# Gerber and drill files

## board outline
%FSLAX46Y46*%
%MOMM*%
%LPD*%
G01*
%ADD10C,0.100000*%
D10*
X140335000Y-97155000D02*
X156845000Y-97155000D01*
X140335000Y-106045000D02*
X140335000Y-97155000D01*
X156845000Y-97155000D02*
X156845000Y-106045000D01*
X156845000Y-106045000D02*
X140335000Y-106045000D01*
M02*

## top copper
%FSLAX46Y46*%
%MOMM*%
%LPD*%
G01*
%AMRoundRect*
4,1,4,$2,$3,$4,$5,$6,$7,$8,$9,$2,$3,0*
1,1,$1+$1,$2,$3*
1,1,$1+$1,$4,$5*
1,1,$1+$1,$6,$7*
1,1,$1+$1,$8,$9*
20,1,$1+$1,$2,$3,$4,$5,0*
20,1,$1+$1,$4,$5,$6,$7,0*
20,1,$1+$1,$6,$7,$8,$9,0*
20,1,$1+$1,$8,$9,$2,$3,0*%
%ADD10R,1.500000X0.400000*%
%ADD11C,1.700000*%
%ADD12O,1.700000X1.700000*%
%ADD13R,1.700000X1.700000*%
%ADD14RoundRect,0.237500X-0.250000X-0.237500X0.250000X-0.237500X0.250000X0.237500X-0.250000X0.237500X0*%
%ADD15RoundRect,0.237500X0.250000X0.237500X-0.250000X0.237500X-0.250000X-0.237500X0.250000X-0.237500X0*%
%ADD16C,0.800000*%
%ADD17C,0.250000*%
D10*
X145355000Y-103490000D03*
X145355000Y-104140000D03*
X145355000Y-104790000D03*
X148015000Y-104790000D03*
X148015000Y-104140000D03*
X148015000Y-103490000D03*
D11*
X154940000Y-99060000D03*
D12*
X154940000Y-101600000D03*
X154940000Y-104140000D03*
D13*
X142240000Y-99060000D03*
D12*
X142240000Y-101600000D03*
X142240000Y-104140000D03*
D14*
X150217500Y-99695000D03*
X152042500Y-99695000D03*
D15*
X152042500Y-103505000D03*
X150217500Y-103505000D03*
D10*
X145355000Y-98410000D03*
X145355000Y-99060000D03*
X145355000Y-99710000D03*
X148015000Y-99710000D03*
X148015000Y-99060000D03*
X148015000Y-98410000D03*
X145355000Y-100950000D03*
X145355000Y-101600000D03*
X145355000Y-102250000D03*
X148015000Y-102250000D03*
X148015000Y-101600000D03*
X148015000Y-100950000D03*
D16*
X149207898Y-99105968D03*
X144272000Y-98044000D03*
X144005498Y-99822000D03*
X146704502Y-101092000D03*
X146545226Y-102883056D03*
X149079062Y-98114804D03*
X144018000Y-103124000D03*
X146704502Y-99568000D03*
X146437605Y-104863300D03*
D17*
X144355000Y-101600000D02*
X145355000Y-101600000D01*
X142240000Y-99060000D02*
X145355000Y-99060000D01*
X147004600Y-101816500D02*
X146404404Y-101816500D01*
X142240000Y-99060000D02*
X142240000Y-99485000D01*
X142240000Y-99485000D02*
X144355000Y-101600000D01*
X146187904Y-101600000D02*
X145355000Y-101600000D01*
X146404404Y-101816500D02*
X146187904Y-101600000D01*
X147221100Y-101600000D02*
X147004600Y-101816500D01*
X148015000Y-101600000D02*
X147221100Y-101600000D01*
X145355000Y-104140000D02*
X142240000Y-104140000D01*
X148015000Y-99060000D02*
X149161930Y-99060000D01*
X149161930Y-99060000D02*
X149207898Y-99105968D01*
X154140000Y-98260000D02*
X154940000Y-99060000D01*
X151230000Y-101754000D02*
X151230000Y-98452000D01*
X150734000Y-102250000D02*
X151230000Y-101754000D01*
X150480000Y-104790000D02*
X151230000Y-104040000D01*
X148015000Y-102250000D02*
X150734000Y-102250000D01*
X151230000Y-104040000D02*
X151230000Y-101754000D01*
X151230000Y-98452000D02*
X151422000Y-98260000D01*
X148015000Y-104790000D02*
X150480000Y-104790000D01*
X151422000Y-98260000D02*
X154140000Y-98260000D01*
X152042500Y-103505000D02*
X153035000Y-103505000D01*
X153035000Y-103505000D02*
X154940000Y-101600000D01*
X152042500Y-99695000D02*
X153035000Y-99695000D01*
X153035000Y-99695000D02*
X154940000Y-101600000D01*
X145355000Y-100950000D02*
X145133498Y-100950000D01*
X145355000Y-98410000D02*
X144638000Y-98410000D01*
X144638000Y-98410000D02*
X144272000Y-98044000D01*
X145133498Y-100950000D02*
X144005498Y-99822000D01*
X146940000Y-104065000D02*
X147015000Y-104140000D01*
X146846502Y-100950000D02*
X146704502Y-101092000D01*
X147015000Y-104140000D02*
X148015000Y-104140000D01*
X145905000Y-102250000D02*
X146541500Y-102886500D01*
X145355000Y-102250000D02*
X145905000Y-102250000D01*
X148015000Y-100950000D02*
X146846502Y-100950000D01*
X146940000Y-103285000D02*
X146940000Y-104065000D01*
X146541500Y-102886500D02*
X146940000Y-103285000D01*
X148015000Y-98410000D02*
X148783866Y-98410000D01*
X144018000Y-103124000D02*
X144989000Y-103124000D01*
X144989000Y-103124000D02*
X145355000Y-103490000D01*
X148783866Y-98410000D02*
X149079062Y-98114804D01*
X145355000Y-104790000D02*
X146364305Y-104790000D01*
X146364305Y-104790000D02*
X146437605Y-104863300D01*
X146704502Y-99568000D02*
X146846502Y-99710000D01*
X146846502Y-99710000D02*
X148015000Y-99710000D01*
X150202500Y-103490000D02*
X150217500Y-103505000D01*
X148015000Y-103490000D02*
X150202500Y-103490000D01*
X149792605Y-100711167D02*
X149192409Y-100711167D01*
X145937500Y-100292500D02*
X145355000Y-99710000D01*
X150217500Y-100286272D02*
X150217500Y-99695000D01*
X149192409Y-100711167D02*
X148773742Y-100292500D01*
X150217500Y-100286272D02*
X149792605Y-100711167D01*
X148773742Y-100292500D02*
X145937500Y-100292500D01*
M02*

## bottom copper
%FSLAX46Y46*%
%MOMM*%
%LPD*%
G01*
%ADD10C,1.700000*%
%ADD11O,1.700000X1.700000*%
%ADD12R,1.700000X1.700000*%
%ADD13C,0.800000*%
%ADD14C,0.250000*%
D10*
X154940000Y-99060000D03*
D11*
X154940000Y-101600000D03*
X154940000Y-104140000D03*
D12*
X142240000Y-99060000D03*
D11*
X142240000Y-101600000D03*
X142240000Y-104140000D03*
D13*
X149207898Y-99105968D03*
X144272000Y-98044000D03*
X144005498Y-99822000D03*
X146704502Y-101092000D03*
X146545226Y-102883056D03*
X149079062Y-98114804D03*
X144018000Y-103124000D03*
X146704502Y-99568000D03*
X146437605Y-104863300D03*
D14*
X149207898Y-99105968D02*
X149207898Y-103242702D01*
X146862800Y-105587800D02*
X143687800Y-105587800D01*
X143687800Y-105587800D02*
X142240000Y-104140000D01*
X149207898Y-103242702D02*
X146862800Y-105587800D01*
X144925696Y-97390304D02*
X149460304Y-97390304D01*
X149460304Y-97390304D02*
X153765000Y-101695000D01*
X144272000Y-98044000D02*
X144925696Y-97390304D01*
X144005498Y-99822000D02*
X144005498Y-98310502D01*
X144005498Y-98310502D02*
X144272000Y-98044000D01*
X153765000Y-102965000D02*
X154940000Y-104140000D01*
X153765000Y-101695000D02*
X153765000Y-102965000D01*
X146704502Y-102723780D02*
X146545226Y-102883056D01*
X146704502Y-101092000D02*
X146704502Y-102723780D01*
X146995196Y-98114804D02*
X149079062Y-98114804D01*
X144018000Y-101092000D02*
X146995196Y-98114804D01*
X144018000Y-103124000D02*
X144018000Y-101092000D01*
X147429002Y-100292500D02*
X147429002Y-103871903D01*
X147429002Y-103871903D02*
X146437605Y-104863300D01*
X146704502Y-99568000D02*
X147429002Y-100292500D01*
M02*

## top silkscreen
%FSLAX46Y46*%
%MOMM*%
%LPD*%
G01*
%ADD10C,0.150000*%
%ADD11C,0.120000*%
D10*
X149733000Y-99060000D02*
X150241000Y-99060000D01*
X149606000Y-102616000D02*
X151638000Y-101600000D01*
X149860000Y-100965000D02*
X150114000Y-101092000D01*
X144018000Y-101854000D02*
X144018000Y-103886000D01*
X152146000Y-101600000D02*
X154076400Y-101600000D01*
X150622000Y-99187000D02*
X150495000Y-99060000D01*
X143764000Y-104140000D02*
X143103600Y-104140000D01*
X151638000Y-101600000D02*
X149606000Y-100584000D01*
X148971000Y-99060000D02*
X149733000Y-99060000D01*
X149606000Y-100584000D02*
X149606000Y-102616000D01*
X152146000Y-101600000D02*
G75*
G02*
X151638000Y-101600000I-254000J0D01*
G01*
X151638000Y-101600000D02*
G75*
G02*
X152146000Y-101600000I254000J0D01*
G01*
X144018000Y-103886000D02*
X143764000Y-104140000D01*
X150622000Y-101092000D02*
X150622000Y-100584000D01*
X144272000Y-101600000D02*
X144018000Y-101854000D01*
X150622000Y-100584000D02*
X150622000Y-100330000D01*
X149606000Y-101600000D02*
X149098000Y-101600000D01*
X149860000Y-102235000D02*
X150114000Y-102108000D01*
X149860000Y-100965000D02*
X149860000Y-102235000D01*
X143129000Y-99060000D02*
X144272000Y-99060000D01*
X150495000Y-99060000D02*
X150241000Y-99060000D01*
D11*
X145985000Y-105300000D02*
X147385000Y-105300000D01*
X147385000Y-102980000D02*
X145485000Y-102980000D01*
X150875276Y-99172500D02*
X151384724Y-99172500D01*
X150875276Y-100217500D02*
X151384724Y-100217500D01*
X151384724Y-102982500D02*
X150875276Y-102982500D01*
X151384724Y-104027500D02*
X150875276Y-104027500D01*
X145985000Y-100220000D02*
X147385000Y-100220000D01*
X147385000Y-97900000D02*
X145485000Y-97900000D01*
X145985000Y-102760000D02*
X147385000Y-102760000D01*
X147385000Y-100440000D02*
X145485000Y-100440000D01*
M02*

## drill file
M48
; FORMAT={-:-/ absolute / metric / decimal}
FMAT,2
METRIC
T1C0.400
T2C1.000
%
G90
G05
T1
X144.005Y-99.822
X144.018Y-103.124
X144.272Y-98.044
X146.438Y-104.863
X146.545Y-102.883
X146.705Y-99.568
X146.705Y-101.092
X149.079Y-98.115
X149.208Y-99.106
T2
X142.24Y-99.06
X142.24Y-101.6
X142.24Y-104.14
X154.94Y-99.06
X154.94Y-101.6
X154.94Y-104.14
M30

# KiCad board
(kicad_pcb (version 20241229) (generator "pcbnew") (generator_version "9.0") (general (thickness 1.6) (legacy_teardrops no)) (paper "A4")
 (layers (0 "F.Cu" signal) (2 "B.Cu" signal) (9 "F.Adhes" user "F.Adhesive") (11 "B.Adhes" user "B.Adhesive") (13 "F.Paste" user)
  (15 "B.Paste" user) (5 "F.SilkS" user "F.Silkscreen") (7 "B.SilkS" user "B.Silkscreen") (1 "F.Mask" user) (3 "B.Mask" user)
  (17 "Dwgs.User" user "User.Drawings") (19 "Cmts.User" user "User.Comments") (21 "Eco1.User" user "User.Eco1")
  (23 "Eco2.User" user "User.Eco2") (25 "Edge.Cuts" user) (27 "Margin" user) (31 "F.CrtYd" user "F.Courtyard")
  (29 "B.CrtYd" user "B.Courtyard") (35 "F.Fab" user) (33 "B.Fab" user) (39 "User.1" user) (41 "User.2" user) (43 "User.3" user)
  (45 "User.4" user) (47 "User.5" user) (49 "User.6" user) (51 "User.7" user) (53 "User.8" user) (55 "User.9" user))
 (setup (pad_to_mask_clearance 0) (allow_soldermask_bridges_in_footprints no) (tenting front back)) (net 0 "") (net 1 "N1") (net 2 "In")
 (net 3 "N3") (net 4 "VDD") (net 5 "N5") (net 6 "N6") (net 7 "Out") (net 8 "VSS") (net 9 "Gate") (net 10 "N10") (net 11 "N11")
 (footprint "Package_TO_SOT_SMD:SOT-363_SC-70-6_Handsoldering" (layer "F.Cu") (at 146.685 104.14)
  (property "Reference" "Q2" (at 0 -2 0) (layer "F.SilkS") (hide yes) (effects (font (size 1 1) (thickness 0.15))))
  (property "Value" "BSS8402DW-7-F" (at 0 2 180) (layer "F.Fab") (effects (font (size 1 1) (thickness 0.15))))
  (fp_line (start -0.7 1.16) (end 0.7 1.16) (stroke (width 0.12) (type solid)) (layer "F.SilkS"))
  (fp_line (start 0.7 -1.16) (end -1.2 -1.16) (stroke (width 0.12) (type solid)) (layer "F.SilkS"))
  (pad "1" smd rect (at -1.33 -0.65) (size 1.5 0.4) (layers "F.Cu" "F.Mask" "F.Paste") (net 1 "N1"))
  (pad "2" smd rect (at -1.33 0) (size 1.5 0.4) (layers "F.Cu" "F.Mask" "F.Paste") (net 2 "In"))
  (pad "3" smd rect (at -1.33 0.65) (size 1.5 0.4) (layers "F.Cu" "F.Mask" "F.Paste") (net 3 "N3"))
  (pad "4" smd rect (at 1.33 0.65) (size 1.5 0.4) (layers "F.Cu" "F.Mask" "F.Paste") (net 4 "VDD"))
  (pad "5" smd rect (at 1.33 0) (size 1.5 0.4) (layers "F.Cu" "F.Mask" "F.Paste") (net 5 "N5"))
  (pad "6" smd rect (at 1.33 -0.65) (size 1.5 0.4) (layers "F.Cu" "F.Mask" "F.Paste") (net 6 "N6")))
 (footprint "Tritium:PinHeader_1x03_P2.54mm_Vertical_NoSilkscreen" (layer "F.Cu") (at 154.94 99.06)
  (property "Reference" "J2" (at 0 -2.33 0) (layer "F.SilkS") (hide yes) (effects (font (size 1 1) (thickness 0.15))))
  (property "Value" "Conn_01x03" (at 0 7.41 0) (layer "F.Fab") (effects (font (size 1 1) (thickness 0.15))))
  (pad "1" thru_hole circle (at 0 0) (size 1.7 1.7) (drill 1) (layers "*.Cu" "*.Mask") (remove_unused_layers no) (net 4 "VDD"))
  (pad "2" thru_hole oval (at 0 2.54) (size 1.7 1.7) (drill 1) (layers "*.Cu" "*.Mask") (remove_unused_layers no) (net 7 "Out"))
  (pad "3" thru_hole oval (at 0 5.08) (size 1.7 1.7) (drill 1) (layers "*.Cu" "*.Mask") (remove_unused_layers no) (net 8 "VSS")))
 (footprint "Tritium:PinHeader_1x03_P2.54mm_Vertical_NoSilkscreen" (layer "F.Cu") (at 142.24 99.06)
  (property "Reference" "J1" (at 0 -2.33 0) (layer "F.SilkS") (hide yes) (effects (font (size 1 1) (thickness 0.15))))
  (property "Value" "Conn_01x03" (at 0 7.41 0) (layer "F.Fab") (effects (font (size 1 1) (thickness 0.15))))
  (pad "1" thru_hole rect (at 0 0) (size 1.7 1.7) (drill 1) (layers "*.Cu" "*.Mask") (remove_unused_layers no) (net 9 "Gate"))
  (pad "2" thru_hole oval (at 0 2.54) (size 1.7 1.7) (drill 1) (layers "*.Cu" "*.Mask") (remove_unused_layers no) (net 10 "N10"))
  (pad "3" thru_hole oval (at 0 5.08) (size 1.7 1.7) (drill 1) (layers "*.Cu" "*.Mask") (remove_unused_layers no) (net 2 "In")))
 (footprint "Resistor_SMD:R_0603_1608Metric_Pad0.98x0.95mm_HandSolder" (layer "F.Cu") (at 151.13 99.695)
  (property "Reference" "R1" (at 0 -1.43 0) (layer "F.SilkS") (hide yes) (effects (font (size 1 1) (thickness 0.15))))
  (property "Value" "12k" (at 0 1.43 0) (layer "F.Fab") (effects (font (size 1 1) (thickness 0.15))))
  (fp_line (start -0.254724 -0.5225) (end 0.254724 -0.5225) (stroke (width 0.12) (type solid)) (layer "F.SilkS"))
  (fp_line (start -0.254724 0.5225) (end 0.254724 0.5225) (stroke (width 0.12) (type solid)) (layer "F.SilkS"))
  (pad "1" smd roundrect (at -0.9125 0) (size 0.975 0.95) (layers "F.Cu" "F.Mask" "F.Paste") (roundrect_rratio 0.25) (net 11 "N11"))
  (pad "2" smd roundrect (at 0.9125 0) (size 0.975 0.95) (layers "F.Cu" "F.Mask" "F.Paste") (roundrect_rratio 0.25) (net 7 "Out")))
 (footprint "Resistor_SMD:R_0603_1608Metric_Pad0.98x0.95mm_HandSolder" (layer "F.Cu") (at 151.13 103.505 180)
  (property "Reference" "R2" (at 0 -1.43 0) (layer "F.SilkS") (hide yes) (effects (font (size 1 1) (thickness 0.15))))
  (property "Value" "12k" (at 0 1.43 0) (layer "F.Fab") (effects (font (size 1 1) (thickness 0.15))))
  (fp_line (start -0.254724 0.5225) (end 0.254724 0.5225) (stroke (width 0.12) (type solid)) (layer "F.SilkS"))
  (fp_line (start -0.254724 -0.5225) (end 0.254724 -0.5225) (stroke (width 0.12) (type solid)) (layer "F.SilkS"))
  (pad "1" smd roundrect (at -0.9125 0 180) (size 0.975 0.95) (layers "F.Cu" "F.Mask" "F.Paste") (roundrect_rratio 0.25) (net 7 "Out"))
  (pad "2" smd roundrect (at 0.9125 0 180) (size 0.975 0.95) (layers "F.Cu" "F.Mask" "F.Paste") (roundrect_rratio 0.25) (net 6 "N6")))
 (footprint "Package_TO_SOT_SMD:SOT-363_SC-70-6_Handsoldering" (layer "F.Cu") (at 146.685 99.06)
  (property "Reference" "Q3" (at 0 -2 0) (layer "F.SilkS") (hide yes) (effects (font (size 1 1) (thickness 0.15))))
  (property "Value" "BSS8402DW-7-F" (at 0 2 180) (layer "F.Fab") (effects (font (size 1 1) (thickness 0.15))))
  (fp_line (start -0.7 1.16) (end 0.7 1.16) (stroke (width 0.12) (type solid)) (layer "F.SilkS"))
  (fp_line (start 0.7 -1.16) (end -1.2 -1.16) (stroke (width 0.12) (type solid)) (layer "F.SilkS"))
  (pad "1" smd rect (at -1.33 -0.65) (size 1.5 0.4) (layers "F.Cu" "F.Mask" "F.Paste") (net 8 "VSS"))
  (pad "2" smd rect (at -1.33 0) (size 1.5 0.4) (layers "F.Cu" "F.Mask" "F.Paste") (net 9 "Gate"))
  (pad "3" smd rect (at -1.33 0.65) (size 1.5 0.4) (layers "F.Cu" "F.Mask" "F.Paste") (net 11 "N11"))
  (pad "4" smd rect (at 1.33 0.65) (size 1.5 0.4) (layers "F.Cu" "F.Mask" "F.Paste") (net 3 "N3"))
  (pad "5" smd rect (at 1.33 0) (size 1.5 0.4) (layers "F.Cu" "F.Mask" "F.Paste") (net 2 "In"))
  (pad "6" smd rect (at 1.33 -0.65) (size 1.5 0.4) (layers "F.Cu" "F.Mask" "F.Paste") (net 1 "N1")))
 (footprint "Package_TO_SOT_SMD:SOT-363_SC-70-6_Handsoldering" (layer "F.Cu") (at 146.685 101.6)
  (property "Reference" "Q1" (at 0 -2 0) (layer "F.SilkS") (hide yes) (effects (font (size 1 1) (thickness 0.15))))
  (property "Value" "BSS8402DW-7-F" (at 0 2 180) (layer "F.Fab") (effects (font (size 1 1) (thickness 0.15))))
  (fp_line (start -0.7 1.16) (end 0.7 1.16) (stroke (width 0.12) (type solid)) (layer "F.SilkS"))
  (fp_line (start 0.7 -1.16) (end -1.2 -1.16) (stroke (width 0.12) (type solid)) (layer "F.SilkS"))
  (pad "1" smd rect (at -1.33 -0.65) (size 1.5 0.4) (layers "F.Cu" "F.Mask" "F.Paste") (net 8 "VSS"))
  (pad "2" smd rect (at -1.33 0) (size 1.5 0.4) (layers "F.Cu" "F.Mask" "F.Paste") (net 9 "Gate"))
  (pad "3" smd rect (at -1.33 0.65) (size 1.5 0.4) (layers "F.Cu" "F.Mask" "F.Paste") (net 5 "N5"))
  (pad "4" smd rect (at 1.33 0.65) (size 1.5 0.4) (layers "F.Cu" "F.Mask" "F.Paste") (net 4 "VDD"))
  (pad "5" smd rect (at 1.33 0) (size 1.5 0.4) (layers "F.Cu" "F.Mask" "F.Paste") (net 9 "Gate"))
  (pad "6" smd rect (at 1.33 -0.65) (size 1.5 0.4) (layers "F.Cu" "F.Mask" "F.Paste") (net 5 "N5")))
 (gr_line (start 149.733 99.06) (end 150.241 99.06) (stroke (width 0.15) (type solid)) (layer "F.SilkS"))
 (gr_line (start 149.606 102.616) (end 151.638 101.6) (stroke (width 0.15) (type solid)) (layer "F.SilkS"))
 (gr_line (start 149.86 100.965) (end 150.114 101.092) (stroke (width 0.15) (type solid)) (layer "F.SilkS"))
 (gr_line (start 144.018 101.854) (end 144.018 103.886) (stroke (width 0.15) (type solid)) (layer "F.SilkS"))
 (gr_line (start 152.146 101.6) (end 154.0764 101.6) (stroke (width 0.15) (type solid)) (layer "F.SilkS"))
 (gr_line (start 150.622 99.187) (end 150.495 99.06) (stroke (width 0.15) (type solid)) (layer "F.SilkS"))
 (gr_line (start 143.764 104.14) (end 143.1036 104.14) (stroke (width 0.15) (type solid)) (layer "F.SilkS"))
 (gr_line (start 151.638 101.6) (end 149.606 100.584) (stroke (width 0.15) (type solid)) (layer "F.SilkS"))
 (gr_line (start 148.971 99.06) (end 149.733 99.06) (stroke (width 0.15) (type solid)) (layer "F.SilkS"))
 (gr_line (start 149.606 100.584) (end 149.606 102.616) (stroke (width 0.15) (type solid)) (layer "F.SilkS"))
 (gr_circle (center 151.892 101.6) (end 152.146 101.6) (stroke (width 0.15) (type solid)) (fill no) (layer "F.SilkS"))
 (gr_line (start 144.018 103.886) (end 143.764 104.14) (stroke (width 0.15) (type solid)) (layer "F.SilkS"))
 (gr_line (start 150.622 101.092) (end 150.622 100.584) (stroke (width 0.15) (type solid)) (layer "F.SilkS"))
 (gr_line (start 144.272 101.6) (end 144.018 101.854) (stroke (width 0.15) (type solid)) (layer "F.SilkS"))
 (gr_line (start 150.622 100.584) (end 150.622 100.33) (stroke (width 0.15) (type solid)) (layer "F.SilkS"))
 (gr_line (start 149.606 101.6) (end 149.098 101.6) (stroke (width 0.15) (type solid)) (layer "F.SilkS"))
 (gr_line (start 149.86 102.235) (end 150.114 102.108) (stroke (width 0.15) (type solid)) (layer "F.SilkS"))
 (gr_line (start 149.86 100.965) (end 149.86 102.235) (stroke (width 0.15) (type solid)) (layer "F.SilkS"))
 (gr_line (start 143.129 99.06) (end 144.272 99.06) (stroke (width 0.15) (type solid)) (layer "F.SilkS"))
 (gr_line (start 150.495 99.06) (end 150.241 99.06) (stroke (width 0.15) (type solid)) (layer "F.SilkS"))
 (gr_line (start 140.335 97.155) (end 156.845 97.155) (stroke (width 0.1) (type solid)) (layer "Edge.Cuts"))
 (gr_line (start 140.335 106.045) (end 140.335 97.155) (stroke (width 0.1) (type solid)) (layer "Edge.Cuts"))
 (gr_line (start 156.845 97.155) (end 156.845 106.045) (stroke (width 0.1) (type solid)) (layer "Edge.Cuts"))
 (gr_line (start 156.845 106.045) (end 140.335 106.045) (stroke (width 0.1) (type solid)) (layer "Edge.Cuts"))
 (segment (start 144.355 101.6) (end 145.355 101.6) (width 0.25) (layer "F.Cu") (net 9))
 (segment (start 142.24 99.06) (end 145.355 99.06) (width 0.25) (layer "F.Cu") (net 9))
 (segment (start 147.0046 101.8165) (end 146.404404 101.8165) (width 0.25) (layer "F.Cu") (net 9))
 (segment (start 142.24 99.06) (end 142.24 99.485) (width 0.25) (layer "F.Cu") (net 9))
 (segment (start 142.24 99.485) (end 144.355 101.6) (width 0.25) (layer "F.Cu") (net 9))
 (segment (start 146.187904 101.6) (end 145.355 101.6) (width 0.25) (layer "F.Cu") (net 9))
 (segment (start 146.404404 101.8165) (end 146.187904 101.6) (width 0.25) (layer "F.Cu") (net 9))
 (segment (start 147.2211 101.6) (end 147.0046 101.8165) (width 0.25) (layer "F.Cu") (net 9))
 (segment (start 148.015 101.6) (end 147.2211 101.6) (width 0.25) (layer "F.Cu") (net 9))
 (segment (start 145.355 104.14) (end 142.24 104.14) (width 0.25) (layer "F.Cu") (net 2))
 (segment (start 148.015 99.06) (end 149.16193 99.06) (width 0.25) (layer "F.Cu") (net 2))
 (segment (start 149.16193 99.06) (end 149.207898 99.105968) (width 0.25) (layer "F.Cu") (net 2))
 (via (at 149.207898 99.105968) (size 0.8) (drill 0.4) (layers "F.Cu" "B.Cu") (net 2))
 (segment (start 149.207898 99.105968) (end 149.207898 103.242702) (width 0.25) (layer "B.Cu") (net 2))
 (segment (start 146.8628 105.5878) (end 143.6878 105.5878) (width 0.25) (layer "B.Cu") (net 2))
 (segment (start 143.6878 105.5878) (end 142.24 104.14) (width 0.25) (layer "B.Cu") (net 2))
 (segment (start 149.207898 103.242702) (end 146.8628 105.5878) (width 0.25) (layer "B.Cu") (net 2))
 (segment (start 154.14 98.26) (end 154.94 99.06) (width 0.25) (layer "F.Cu") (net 4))
 (segment (start 151.23 101.754) (end 151.23 98.452) (width 0.25) (layer "F.Cu") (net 4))
 (segment (start 150.734 102.25) (end 151.23 101.754) (width 0.25) (layer "F.Cu") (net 4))
 (segment (start 150.48 104.79) (end 151.23 104.04) (width 0.25) (layer "F.Cu") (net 4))
 (segment (start 148.015 102.25) (end 150.734 102.25) (width 0.25) (layer "F.Cu") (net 4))
 (segment (start 151.23 104.04) (end 151.23 101.754) (width 0.25) (layer "F.Cu") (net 4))
 (segment (start 151.23 98.452) (end 151.422 98.26) (width 0.25) (layer "F.Cu") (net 4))
 (segment (start 148.015 104.79) (end 150.48 104.79) (width 0.25) (layer "F.Cu") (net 4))
 (segment (start 151.422 98.26) (end 154.14 98.26) (width 0.25) (layer "F.Cu") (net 4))
 (segment (start 152.0425 103.505) (end 153.035 103.505) (width 0.25) (layer "F.Cu") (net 7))
 (segment (start 153.035 103.505) (end 154.94 101.6) (width 0.25) (layer "F.Cu") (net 7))
 (segment (start 152.0425 99.695) (end 153.035 99.695) (width 0.25) (layer "F.Cu") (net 7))
 (segment (start 153.035 99.695) (end 154.94 101.6) (width 0.25) (layer "F.Cu") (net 7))
 (segment (start 145.355 100.95) (end 145.133498 100.95) (width 0.25) (layer "F.Cu") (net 8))
 (segment (start 145.355 98.41) (end 144.638 98.41) (width 0.25) (layer "F.Cu") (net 8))
 (segment (start 144.638 98.41) (end 144.272 98.044) (width 0.25) (layer "F.Cu") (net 8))
 (segment (start 145.133498 100.95) (end 144.005498 99.822) (width 0.25) (layer "F.Cu") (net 8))
 (via (at 144.272 98.044) (size 0.8) (drill 0.4) (layers "F.Cu" "B.Cu") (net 8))
 (via (at 144.005498 99.822) (size 0.8) (drill 0.4) (layers "F.Cu" "B.Cu") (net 8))
 (segment (start 144.925696 97.390304) (end 149.460304 97.390304) (width 0.25) (layer "B.Cu") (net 8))
 (segment (start 149.460304 97.390304) (end 153.765 101.695) (width 0.25) (layer "B.Cu") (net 8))
 (segment (start 144.272 98.044) (end 144.925696 97.390304) (width 0.25) (layer "B.Cu") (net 8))
 (segment (start 144.005498 99.822) (end 144.005498 98.310502) (width 0.25) (layer "B.Cu") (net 8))
 (segment (start 144.005498 98.310502) (end 144.272 98.044) (width 0.25) (layer "B.Cu") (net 8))
 (segment (start 153.765 102.965) (end 154.94 104.14) (width 0.25) (layer "B.Cu") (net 8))
 (segment (start 153.765 101.695) (end 153.765 102.965) (width 0.25) (layer "B.Cu") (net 8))
 (segment (start 146.94 104.065) (end 147.015 104.14) (width 0.25) (layer "F.Cu") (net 5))
 (segment (start 146.846502 100.95) (end 146.704502 101.092) (width 0.25) (layer "F.Cu") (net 5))
 (segment (start 147.015 104.14) (end 148.015 104.14) (width 0.25) (layer "F.Cu") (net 5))
 (segment (start 145.905 102.25) (end 146.5415 102.8865) (width 0.25) (layer "F.Cu") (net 5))
 (segment (start 145.355 102.25) (end 145.905 102.25) (width 0.25) (layer "F.Cu") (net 5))
 (segment (start 148.015 100.95) (end 146.846502 100.95) (width 0.25) (layer "F.Cu") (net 5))
 (segment (start 146.94 103.285) (end 146.94 104.065) (width 0.25) (layer "F.Cu") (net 5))
 (segment (start 146.5415 102.8865) (end 146.94 103.285) (width 0.25) (layer "F.Cu") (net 5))
 (via (at 146.704502 101.092) (size 0.8) (drill 0.4) (layers "F.Cu" "B.Cu") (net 5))
 (via (at 146.545226 102.883056) (size 0.8) (drill 0.4) (layers "F.Cu" "B.Cu") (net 5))
 (segment (start 146.704502 102.72378) (end 146.545226 102.883056) (width 0.25) (layer "B.Cu") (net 5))
 (segment (start 146.704502 101.092) (end 146.704502 102.72378) (width 0.25) (layer "B.Cu") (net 5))
 (segment (start 148.015 98.41) (end 148.783866 98.41) (width 0.25) (layer "F.Cu") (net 1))
 (segment (start 144.018 103.124) (end 144.989 103.124) (width 0.25) (layer "F.Cu") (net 1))
 (segment (start 144.989 103.124) (end 145.355 103.49) (width 0.25) (layer "F.Cu") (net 1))
 (segment (start 148.783866 98.41) (end 149.079062 98.114804) (width 0.25) (layer "F.Cu") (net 1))
 (via (at 149.079062 98.114804) (size 0.8) (drill 0.4) (layers "F.Cu" "B.Cu") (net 1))
 (via (at 144.018 103.124) (size 0.8) (drill 0.4) (layers "F.Cu" "B.Cu") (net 1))
 (segment (start 146.995196 98.114804) (end 149.079062 98.114804) (width 0.25) (layer "B.Cu") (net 1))
 (segment (start 144.018 101.092) (end 146.995196 98.114804) (width 0.25) (layer "B.Cu") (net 1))
 (segment (start 144.018 103.124) (end 144.018 101.092) (width 0.25) (layer "B.Cu") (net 1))
 (segment (start 145.355 104.79) (end 146.364305 104.79) (width 0.25) (layer "F.Cu") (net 3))
 (segment (start 146.364305 104.79) (end 146.437605 104.8633) (width 0.25) (layer "F.Cu") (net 3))
 (segment (start 146.704502 99.568) (end 146.846502 99.71) (width 0.25) (layer "F.Cu") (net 3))
 (segment (start 146.846502 99.71) (end 148.015 99.71) (width 0.25) (layer "F.Cu") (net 3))
 (via (at 146.704502 99.568) (size 0.8) (drill 0.4) (layers "F.Cu" "B.Cu") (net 3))
 (via (at 146.437605 104.8633) (size 0.8) (drill 0.4) (layers "F.Cu" "B.Cu") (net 3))
 (segment (start 147.429002 100.2925) (end 147.429002 103.871903) (width 0.25) (layer "B.Cu") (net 3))
 (segment (start 147.429002 103.871903) (end 146.437605 104.8633) (width 0.25) (layer "B.Cu") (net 3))
 (segment (start 146.704502 99.568) (end 147.429002 100.2925) (width 0.25) (layer "B.Cu") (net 3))
 (segment (start 150.2025 103.49) (end 150.2175 103.505) (width 0.25) (layer "F.Cu") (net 6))
 (segment (start 148.015 103.49) (end 150.2025 103.49) (width 0.25) (layer "F.Cu") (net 6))
 (segment (start 149.792605 100.711167) (end 149.192409 100.711167) (width 0.25) (layer "F.Cu") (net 11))
 (segment (start 145.9375 100.2925) (end 145.355 99.71) (width 0.25) (layer "F.Cu") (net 11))
 (segment (start 150.2175 100.286272) (end 150.2175 99.695) (width 0.25) (layer "F.Cu") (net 11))
 (segment (start 149.192409 100.711167) (end 148.773742 100.2925) (width 0.25) (layer "F.Cu") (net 11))
 (segment (start 150.2175 100.286272) (end 149.792605 100.711167) (width 0.25) (layer "F.Cu") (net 11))
 (segment (start 148.773742 100.2925) (end 145.9375 100.2925) (width 0.25) (layer "F.Cu") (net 11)))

